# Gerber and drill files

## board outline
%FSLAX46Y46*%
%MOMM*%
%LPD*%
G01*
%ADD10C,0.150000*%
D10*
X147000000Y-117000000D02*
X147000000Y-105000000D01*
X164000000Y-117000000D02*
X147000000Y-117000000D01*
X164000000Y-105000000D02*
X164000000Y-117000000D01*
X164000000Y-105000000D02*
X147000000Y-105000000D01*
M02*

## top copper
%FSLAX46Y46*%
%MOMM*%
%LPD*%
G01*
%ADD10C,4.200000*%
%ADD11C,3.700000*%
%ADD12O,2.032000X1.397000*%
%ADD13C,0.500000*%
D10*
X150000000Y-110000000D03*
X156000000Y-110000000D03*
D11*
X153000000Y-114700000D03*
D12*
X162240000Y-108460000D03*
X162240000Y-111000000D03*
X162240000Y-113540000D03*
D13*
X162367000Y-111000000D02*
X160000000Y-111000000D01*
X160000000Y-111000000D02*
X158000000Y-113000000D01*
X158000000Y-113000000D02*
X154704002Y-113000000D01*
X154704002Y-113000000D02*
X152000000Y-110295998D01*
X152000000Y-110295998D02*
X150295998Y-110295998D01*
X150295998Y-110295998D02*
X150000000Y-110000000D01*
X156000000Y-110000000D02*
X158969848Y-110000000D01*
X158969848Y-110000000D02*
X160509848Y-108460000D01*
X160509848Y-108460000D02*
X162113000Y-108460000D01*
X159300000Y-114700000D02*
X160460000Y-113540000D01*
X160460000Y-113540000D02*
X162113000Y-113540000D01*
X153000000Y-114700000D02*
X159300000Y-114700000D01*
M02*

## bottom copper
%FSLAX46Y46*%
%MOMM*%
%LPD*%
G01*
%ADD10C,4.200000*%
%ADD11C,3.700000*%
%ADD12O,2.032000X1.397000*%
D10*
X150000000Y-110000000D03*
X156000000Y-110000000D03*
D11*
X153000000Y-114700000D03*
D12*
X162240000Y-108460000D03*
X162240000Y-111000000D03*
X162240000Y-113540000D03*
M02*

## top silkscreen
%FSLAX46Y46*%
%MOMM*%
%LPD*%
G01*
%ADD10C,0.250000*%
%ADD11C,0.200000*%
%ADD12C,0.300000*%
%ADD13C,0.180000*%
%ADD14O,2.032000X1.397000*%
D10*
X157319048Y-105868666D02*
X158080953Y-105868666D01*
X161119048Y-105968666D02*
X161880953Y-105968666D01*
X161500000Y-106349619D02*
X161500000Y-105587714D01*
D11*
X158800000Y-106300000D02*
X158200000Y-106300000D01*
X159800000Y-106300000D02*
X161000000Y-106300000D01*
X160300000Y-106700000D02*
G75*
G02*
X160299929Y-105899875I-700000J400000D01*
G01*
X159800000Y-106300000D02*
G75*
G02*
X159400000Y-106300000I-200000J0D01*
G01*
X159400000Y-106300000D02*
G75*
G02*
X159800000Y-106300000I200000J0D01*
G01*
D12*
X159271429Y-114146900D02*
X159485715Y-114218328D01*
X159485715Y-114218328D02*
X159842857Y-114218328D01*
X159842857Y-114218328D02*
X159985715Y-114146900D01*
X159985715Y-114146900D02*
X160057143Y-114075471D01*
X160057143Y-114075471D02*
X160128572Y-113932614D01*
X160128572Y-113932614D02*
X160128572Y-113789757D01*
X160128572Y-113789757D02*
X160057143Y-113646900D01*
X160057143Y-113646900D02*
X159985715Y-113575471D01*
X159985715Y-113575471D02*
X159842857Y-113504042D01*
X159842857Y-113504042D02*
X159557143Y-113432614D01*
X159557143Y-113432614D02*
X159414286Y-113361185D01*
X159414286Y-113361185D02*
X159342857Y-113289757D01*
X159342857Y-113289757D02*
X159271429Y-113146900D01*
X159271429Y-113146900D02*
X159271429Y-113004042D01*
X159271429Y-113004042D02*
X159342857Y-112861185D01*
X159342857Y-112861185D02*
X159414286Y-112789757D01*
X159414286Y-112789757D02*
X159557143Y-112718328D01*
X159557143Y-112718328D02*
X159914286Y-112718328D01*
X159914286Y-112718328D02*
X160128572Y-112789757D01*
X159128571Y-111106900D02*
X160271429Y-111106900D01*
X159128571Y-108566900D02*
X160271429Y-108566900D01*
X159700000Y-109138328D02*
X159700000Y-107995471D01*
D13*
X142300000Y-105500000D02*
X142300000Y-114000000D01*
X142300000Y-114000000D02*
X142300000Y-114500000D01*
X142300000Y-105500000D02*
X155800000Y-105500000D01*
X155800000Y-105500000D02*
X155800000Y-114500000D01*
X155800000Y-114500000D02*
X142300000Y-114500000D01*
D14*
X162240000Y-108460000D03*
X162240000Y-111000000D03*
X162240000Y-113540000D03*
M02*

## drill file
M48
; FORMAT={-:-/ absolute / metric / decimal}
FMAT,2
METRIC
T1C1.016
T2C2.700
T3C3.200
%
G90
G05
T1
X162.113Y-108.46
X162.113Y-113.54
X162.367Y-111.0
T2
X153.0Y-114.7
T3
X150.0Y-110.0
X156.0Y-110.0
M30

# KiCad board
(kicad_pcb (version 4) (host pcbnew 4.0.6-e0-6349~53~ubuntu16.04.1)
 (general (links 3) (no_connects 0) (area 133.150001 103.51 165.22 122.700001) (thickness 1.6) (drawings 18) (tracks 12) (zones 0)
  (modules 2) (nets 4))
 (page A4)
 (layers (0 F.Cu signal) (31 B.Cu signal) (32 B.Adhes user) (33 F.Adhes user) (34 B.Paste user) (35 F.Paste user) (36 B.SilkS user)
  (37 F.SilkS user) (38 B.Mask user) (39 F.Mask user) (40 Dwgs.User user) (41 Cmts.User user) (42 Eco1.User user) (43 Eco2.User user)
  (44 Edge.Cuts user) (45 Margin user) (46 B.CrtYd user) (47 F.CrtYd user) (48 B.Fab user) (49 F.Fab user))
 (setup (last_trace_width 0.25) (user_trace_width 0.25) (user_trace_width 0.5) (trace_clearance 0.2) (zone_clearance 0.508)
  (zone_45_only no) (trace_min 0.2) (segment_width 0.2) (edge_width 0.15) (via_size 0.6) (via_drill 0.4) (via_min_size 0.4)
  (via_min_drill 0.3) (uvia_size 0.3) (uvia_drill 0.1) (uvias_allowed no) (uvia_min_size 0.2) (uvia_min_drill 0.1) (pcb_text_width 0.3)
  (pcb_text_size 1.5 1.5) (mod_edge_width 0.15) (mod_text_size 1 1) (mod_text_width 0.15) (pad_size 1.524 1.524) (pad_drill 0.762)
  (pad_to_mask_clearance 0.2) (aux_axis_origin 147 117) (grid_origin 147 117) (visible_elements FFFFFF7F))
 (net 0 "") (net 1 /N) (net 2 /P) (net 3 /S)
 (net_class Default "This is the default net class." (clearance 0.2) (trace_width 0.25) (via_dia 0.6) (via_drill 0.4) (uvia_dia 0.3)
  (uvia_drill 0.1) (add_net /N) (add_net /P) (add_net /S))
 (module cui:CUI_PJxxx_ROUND (layer F.Cu) (at 142.3 110)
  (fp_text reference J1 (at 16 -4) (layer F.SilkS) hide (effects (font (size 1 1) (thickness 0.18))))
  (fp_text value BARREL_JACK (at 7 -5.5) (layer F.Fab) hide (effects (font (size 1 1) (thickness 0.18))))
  (fp_line (start 0 -4.5) (end 0 4) (layer F.SilkS) (width 0.18))
  (fp_line (start 0 4) (end 0 4.5) (layer F.SilkS) (width 0.18))
  (fp_line (start 0 -4.5) (end 13.5 -4.5) (layer F.SilkS) (width 0.18))
  (fp_line (start 13.5 -4.5) (end 13.5 4.5) (layer F.SilkS) (width 0.18))
  (fp_line (start 13.5 4.5) (end 0 4.5) (layer F.SilkS) (width 0.18))
  (pad 2 thru_hole circle (at 7.7 0) (size 4.2 4.2) (drill 3.2) (layers *.Cu *.Mask) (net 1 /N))
  (pad 1 thru_hole circle (at 13.7 0) (size 4.2 4.2) (drill 3.2) (layers *.Cu *.Mask) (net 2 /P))
  (pad 3 thru_hole circle (at 10.7 4.7) (size 3.7 3.7) (drill 2.7) (layers *.Cu *.Mask) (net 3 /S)))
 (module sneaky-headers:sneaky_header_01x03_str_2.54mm (layer F.Cu) (at 162.24 108.46 270)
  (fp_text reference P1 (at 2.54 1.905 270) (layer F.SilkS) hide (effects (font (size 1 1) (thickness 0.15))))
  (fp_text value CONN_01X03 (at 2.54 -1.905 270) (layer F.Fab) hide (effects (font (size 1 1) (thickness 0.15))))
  (pad 1 thru_hole oval (at 0 0.127 270) (size 1.397 2.032) (drill 1.016 (offset 0 -0.127)) (layers *.Cu *.Mask F.SilkS) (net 2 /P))
  (pad 2 thru_hole oval (at 2.54 -0.127 270) (size 1.397 2.032) (drill 1.016 (offset 0 0.127)) (layers *.Cu *.Mask F.SilkS) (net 1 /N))
  (pad 3 thru_hole oval (at 5.08 0.127 270) (size 1.397 2.032) (drill 1.016 (offset 0 -0.127)) (layers *.Cu *.Mask F.SilkS) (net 3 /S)))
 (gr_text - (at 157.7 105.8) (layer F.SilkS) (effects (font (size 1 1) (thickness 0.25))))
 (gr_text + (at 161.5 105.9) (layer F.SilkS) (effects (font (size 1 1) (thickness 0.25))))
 (gr_line (start 158.8 106.3) (end 158.2 106.3) (layer F.SilkS) (width 0.2))
 (gr_line (start 159.8 106.3) (end 161 106.3) (layer F.SilkS) (width 0.2))
 (gr_arc (start 159.6 106.3) (end 160.3 106.7) (angle 300.5) (layer F.SilkS) (width 0.2))
 (gr_circle (center 159.6 106.3) (end 159.8 106.3) (layer F.SilkS) (width 0.2))
 (gr_line (start 147 117) (end 147 105) (layer Edge.Cuts) (width 0.15))
 (gr_line (start 164 117) (end 147 117) (layer Edge.Cuts) (width 0.15))
 (gr_line (start 164 105) (end 164 117) (layer Edge.Cuts) (width 0.15))
 (gr_line (start 164 105) (end 147 105) (layer Edge.Cuts) (width 0.15))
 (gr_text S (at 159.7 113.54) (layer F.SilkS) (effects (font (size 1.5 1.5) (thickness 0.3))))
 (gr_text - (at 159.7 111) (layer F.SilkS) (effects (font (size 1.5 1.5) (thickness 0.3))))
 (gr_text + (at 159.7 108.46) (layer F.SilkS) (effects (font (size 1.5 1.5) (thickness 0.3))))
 (segment (start 162.367 111) (end 160 111) (width 0.5) (layer F.Cu) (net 1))
 (segment (start 160 111) (end 158 113) (width 0.5) (layer F.Cu) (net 1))
 (segment (start 158 113) (end 154.704002 113) (width 0.5) (layer F.Cu) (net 1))
 (segment (start 154.704002 113) (end 152 110.295998) (width 0.5) (layer F.Cu) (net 1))
 (segment (start 152 110.295998) (end 150.295998 110.295998) (width 0.5) (layer F.Cu) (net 1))
 (segment (start 150.295998 110.295998) (end 150 110) (width 0.5) (layer F.Cu) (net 1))
 (segment (start 156 110) (end 158.969848 110) (width 0.5) (layer F.Cu) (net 2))
 (segment (start 158.969848 110) (end 160.509848 108.46) (width 0.5) (layer F.Cu) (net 2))
 (segment (start 160.509848 108.46) (end 162.113 108.46) (width 0.5) (layer F.Cu) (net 2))
 (segment (start 159.3 114.7) (end 160.46 113.54) (width 0.5) (layer F.Cu) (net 3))
 (segment (start 160.46 113.54) (end 162.113 113.54) (width 0.5) (layer F.Cu) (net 3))
 (segment (start 153 114.7) (end 159.3 114.7) (width 0.5) (layer F.Cu) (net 3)))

